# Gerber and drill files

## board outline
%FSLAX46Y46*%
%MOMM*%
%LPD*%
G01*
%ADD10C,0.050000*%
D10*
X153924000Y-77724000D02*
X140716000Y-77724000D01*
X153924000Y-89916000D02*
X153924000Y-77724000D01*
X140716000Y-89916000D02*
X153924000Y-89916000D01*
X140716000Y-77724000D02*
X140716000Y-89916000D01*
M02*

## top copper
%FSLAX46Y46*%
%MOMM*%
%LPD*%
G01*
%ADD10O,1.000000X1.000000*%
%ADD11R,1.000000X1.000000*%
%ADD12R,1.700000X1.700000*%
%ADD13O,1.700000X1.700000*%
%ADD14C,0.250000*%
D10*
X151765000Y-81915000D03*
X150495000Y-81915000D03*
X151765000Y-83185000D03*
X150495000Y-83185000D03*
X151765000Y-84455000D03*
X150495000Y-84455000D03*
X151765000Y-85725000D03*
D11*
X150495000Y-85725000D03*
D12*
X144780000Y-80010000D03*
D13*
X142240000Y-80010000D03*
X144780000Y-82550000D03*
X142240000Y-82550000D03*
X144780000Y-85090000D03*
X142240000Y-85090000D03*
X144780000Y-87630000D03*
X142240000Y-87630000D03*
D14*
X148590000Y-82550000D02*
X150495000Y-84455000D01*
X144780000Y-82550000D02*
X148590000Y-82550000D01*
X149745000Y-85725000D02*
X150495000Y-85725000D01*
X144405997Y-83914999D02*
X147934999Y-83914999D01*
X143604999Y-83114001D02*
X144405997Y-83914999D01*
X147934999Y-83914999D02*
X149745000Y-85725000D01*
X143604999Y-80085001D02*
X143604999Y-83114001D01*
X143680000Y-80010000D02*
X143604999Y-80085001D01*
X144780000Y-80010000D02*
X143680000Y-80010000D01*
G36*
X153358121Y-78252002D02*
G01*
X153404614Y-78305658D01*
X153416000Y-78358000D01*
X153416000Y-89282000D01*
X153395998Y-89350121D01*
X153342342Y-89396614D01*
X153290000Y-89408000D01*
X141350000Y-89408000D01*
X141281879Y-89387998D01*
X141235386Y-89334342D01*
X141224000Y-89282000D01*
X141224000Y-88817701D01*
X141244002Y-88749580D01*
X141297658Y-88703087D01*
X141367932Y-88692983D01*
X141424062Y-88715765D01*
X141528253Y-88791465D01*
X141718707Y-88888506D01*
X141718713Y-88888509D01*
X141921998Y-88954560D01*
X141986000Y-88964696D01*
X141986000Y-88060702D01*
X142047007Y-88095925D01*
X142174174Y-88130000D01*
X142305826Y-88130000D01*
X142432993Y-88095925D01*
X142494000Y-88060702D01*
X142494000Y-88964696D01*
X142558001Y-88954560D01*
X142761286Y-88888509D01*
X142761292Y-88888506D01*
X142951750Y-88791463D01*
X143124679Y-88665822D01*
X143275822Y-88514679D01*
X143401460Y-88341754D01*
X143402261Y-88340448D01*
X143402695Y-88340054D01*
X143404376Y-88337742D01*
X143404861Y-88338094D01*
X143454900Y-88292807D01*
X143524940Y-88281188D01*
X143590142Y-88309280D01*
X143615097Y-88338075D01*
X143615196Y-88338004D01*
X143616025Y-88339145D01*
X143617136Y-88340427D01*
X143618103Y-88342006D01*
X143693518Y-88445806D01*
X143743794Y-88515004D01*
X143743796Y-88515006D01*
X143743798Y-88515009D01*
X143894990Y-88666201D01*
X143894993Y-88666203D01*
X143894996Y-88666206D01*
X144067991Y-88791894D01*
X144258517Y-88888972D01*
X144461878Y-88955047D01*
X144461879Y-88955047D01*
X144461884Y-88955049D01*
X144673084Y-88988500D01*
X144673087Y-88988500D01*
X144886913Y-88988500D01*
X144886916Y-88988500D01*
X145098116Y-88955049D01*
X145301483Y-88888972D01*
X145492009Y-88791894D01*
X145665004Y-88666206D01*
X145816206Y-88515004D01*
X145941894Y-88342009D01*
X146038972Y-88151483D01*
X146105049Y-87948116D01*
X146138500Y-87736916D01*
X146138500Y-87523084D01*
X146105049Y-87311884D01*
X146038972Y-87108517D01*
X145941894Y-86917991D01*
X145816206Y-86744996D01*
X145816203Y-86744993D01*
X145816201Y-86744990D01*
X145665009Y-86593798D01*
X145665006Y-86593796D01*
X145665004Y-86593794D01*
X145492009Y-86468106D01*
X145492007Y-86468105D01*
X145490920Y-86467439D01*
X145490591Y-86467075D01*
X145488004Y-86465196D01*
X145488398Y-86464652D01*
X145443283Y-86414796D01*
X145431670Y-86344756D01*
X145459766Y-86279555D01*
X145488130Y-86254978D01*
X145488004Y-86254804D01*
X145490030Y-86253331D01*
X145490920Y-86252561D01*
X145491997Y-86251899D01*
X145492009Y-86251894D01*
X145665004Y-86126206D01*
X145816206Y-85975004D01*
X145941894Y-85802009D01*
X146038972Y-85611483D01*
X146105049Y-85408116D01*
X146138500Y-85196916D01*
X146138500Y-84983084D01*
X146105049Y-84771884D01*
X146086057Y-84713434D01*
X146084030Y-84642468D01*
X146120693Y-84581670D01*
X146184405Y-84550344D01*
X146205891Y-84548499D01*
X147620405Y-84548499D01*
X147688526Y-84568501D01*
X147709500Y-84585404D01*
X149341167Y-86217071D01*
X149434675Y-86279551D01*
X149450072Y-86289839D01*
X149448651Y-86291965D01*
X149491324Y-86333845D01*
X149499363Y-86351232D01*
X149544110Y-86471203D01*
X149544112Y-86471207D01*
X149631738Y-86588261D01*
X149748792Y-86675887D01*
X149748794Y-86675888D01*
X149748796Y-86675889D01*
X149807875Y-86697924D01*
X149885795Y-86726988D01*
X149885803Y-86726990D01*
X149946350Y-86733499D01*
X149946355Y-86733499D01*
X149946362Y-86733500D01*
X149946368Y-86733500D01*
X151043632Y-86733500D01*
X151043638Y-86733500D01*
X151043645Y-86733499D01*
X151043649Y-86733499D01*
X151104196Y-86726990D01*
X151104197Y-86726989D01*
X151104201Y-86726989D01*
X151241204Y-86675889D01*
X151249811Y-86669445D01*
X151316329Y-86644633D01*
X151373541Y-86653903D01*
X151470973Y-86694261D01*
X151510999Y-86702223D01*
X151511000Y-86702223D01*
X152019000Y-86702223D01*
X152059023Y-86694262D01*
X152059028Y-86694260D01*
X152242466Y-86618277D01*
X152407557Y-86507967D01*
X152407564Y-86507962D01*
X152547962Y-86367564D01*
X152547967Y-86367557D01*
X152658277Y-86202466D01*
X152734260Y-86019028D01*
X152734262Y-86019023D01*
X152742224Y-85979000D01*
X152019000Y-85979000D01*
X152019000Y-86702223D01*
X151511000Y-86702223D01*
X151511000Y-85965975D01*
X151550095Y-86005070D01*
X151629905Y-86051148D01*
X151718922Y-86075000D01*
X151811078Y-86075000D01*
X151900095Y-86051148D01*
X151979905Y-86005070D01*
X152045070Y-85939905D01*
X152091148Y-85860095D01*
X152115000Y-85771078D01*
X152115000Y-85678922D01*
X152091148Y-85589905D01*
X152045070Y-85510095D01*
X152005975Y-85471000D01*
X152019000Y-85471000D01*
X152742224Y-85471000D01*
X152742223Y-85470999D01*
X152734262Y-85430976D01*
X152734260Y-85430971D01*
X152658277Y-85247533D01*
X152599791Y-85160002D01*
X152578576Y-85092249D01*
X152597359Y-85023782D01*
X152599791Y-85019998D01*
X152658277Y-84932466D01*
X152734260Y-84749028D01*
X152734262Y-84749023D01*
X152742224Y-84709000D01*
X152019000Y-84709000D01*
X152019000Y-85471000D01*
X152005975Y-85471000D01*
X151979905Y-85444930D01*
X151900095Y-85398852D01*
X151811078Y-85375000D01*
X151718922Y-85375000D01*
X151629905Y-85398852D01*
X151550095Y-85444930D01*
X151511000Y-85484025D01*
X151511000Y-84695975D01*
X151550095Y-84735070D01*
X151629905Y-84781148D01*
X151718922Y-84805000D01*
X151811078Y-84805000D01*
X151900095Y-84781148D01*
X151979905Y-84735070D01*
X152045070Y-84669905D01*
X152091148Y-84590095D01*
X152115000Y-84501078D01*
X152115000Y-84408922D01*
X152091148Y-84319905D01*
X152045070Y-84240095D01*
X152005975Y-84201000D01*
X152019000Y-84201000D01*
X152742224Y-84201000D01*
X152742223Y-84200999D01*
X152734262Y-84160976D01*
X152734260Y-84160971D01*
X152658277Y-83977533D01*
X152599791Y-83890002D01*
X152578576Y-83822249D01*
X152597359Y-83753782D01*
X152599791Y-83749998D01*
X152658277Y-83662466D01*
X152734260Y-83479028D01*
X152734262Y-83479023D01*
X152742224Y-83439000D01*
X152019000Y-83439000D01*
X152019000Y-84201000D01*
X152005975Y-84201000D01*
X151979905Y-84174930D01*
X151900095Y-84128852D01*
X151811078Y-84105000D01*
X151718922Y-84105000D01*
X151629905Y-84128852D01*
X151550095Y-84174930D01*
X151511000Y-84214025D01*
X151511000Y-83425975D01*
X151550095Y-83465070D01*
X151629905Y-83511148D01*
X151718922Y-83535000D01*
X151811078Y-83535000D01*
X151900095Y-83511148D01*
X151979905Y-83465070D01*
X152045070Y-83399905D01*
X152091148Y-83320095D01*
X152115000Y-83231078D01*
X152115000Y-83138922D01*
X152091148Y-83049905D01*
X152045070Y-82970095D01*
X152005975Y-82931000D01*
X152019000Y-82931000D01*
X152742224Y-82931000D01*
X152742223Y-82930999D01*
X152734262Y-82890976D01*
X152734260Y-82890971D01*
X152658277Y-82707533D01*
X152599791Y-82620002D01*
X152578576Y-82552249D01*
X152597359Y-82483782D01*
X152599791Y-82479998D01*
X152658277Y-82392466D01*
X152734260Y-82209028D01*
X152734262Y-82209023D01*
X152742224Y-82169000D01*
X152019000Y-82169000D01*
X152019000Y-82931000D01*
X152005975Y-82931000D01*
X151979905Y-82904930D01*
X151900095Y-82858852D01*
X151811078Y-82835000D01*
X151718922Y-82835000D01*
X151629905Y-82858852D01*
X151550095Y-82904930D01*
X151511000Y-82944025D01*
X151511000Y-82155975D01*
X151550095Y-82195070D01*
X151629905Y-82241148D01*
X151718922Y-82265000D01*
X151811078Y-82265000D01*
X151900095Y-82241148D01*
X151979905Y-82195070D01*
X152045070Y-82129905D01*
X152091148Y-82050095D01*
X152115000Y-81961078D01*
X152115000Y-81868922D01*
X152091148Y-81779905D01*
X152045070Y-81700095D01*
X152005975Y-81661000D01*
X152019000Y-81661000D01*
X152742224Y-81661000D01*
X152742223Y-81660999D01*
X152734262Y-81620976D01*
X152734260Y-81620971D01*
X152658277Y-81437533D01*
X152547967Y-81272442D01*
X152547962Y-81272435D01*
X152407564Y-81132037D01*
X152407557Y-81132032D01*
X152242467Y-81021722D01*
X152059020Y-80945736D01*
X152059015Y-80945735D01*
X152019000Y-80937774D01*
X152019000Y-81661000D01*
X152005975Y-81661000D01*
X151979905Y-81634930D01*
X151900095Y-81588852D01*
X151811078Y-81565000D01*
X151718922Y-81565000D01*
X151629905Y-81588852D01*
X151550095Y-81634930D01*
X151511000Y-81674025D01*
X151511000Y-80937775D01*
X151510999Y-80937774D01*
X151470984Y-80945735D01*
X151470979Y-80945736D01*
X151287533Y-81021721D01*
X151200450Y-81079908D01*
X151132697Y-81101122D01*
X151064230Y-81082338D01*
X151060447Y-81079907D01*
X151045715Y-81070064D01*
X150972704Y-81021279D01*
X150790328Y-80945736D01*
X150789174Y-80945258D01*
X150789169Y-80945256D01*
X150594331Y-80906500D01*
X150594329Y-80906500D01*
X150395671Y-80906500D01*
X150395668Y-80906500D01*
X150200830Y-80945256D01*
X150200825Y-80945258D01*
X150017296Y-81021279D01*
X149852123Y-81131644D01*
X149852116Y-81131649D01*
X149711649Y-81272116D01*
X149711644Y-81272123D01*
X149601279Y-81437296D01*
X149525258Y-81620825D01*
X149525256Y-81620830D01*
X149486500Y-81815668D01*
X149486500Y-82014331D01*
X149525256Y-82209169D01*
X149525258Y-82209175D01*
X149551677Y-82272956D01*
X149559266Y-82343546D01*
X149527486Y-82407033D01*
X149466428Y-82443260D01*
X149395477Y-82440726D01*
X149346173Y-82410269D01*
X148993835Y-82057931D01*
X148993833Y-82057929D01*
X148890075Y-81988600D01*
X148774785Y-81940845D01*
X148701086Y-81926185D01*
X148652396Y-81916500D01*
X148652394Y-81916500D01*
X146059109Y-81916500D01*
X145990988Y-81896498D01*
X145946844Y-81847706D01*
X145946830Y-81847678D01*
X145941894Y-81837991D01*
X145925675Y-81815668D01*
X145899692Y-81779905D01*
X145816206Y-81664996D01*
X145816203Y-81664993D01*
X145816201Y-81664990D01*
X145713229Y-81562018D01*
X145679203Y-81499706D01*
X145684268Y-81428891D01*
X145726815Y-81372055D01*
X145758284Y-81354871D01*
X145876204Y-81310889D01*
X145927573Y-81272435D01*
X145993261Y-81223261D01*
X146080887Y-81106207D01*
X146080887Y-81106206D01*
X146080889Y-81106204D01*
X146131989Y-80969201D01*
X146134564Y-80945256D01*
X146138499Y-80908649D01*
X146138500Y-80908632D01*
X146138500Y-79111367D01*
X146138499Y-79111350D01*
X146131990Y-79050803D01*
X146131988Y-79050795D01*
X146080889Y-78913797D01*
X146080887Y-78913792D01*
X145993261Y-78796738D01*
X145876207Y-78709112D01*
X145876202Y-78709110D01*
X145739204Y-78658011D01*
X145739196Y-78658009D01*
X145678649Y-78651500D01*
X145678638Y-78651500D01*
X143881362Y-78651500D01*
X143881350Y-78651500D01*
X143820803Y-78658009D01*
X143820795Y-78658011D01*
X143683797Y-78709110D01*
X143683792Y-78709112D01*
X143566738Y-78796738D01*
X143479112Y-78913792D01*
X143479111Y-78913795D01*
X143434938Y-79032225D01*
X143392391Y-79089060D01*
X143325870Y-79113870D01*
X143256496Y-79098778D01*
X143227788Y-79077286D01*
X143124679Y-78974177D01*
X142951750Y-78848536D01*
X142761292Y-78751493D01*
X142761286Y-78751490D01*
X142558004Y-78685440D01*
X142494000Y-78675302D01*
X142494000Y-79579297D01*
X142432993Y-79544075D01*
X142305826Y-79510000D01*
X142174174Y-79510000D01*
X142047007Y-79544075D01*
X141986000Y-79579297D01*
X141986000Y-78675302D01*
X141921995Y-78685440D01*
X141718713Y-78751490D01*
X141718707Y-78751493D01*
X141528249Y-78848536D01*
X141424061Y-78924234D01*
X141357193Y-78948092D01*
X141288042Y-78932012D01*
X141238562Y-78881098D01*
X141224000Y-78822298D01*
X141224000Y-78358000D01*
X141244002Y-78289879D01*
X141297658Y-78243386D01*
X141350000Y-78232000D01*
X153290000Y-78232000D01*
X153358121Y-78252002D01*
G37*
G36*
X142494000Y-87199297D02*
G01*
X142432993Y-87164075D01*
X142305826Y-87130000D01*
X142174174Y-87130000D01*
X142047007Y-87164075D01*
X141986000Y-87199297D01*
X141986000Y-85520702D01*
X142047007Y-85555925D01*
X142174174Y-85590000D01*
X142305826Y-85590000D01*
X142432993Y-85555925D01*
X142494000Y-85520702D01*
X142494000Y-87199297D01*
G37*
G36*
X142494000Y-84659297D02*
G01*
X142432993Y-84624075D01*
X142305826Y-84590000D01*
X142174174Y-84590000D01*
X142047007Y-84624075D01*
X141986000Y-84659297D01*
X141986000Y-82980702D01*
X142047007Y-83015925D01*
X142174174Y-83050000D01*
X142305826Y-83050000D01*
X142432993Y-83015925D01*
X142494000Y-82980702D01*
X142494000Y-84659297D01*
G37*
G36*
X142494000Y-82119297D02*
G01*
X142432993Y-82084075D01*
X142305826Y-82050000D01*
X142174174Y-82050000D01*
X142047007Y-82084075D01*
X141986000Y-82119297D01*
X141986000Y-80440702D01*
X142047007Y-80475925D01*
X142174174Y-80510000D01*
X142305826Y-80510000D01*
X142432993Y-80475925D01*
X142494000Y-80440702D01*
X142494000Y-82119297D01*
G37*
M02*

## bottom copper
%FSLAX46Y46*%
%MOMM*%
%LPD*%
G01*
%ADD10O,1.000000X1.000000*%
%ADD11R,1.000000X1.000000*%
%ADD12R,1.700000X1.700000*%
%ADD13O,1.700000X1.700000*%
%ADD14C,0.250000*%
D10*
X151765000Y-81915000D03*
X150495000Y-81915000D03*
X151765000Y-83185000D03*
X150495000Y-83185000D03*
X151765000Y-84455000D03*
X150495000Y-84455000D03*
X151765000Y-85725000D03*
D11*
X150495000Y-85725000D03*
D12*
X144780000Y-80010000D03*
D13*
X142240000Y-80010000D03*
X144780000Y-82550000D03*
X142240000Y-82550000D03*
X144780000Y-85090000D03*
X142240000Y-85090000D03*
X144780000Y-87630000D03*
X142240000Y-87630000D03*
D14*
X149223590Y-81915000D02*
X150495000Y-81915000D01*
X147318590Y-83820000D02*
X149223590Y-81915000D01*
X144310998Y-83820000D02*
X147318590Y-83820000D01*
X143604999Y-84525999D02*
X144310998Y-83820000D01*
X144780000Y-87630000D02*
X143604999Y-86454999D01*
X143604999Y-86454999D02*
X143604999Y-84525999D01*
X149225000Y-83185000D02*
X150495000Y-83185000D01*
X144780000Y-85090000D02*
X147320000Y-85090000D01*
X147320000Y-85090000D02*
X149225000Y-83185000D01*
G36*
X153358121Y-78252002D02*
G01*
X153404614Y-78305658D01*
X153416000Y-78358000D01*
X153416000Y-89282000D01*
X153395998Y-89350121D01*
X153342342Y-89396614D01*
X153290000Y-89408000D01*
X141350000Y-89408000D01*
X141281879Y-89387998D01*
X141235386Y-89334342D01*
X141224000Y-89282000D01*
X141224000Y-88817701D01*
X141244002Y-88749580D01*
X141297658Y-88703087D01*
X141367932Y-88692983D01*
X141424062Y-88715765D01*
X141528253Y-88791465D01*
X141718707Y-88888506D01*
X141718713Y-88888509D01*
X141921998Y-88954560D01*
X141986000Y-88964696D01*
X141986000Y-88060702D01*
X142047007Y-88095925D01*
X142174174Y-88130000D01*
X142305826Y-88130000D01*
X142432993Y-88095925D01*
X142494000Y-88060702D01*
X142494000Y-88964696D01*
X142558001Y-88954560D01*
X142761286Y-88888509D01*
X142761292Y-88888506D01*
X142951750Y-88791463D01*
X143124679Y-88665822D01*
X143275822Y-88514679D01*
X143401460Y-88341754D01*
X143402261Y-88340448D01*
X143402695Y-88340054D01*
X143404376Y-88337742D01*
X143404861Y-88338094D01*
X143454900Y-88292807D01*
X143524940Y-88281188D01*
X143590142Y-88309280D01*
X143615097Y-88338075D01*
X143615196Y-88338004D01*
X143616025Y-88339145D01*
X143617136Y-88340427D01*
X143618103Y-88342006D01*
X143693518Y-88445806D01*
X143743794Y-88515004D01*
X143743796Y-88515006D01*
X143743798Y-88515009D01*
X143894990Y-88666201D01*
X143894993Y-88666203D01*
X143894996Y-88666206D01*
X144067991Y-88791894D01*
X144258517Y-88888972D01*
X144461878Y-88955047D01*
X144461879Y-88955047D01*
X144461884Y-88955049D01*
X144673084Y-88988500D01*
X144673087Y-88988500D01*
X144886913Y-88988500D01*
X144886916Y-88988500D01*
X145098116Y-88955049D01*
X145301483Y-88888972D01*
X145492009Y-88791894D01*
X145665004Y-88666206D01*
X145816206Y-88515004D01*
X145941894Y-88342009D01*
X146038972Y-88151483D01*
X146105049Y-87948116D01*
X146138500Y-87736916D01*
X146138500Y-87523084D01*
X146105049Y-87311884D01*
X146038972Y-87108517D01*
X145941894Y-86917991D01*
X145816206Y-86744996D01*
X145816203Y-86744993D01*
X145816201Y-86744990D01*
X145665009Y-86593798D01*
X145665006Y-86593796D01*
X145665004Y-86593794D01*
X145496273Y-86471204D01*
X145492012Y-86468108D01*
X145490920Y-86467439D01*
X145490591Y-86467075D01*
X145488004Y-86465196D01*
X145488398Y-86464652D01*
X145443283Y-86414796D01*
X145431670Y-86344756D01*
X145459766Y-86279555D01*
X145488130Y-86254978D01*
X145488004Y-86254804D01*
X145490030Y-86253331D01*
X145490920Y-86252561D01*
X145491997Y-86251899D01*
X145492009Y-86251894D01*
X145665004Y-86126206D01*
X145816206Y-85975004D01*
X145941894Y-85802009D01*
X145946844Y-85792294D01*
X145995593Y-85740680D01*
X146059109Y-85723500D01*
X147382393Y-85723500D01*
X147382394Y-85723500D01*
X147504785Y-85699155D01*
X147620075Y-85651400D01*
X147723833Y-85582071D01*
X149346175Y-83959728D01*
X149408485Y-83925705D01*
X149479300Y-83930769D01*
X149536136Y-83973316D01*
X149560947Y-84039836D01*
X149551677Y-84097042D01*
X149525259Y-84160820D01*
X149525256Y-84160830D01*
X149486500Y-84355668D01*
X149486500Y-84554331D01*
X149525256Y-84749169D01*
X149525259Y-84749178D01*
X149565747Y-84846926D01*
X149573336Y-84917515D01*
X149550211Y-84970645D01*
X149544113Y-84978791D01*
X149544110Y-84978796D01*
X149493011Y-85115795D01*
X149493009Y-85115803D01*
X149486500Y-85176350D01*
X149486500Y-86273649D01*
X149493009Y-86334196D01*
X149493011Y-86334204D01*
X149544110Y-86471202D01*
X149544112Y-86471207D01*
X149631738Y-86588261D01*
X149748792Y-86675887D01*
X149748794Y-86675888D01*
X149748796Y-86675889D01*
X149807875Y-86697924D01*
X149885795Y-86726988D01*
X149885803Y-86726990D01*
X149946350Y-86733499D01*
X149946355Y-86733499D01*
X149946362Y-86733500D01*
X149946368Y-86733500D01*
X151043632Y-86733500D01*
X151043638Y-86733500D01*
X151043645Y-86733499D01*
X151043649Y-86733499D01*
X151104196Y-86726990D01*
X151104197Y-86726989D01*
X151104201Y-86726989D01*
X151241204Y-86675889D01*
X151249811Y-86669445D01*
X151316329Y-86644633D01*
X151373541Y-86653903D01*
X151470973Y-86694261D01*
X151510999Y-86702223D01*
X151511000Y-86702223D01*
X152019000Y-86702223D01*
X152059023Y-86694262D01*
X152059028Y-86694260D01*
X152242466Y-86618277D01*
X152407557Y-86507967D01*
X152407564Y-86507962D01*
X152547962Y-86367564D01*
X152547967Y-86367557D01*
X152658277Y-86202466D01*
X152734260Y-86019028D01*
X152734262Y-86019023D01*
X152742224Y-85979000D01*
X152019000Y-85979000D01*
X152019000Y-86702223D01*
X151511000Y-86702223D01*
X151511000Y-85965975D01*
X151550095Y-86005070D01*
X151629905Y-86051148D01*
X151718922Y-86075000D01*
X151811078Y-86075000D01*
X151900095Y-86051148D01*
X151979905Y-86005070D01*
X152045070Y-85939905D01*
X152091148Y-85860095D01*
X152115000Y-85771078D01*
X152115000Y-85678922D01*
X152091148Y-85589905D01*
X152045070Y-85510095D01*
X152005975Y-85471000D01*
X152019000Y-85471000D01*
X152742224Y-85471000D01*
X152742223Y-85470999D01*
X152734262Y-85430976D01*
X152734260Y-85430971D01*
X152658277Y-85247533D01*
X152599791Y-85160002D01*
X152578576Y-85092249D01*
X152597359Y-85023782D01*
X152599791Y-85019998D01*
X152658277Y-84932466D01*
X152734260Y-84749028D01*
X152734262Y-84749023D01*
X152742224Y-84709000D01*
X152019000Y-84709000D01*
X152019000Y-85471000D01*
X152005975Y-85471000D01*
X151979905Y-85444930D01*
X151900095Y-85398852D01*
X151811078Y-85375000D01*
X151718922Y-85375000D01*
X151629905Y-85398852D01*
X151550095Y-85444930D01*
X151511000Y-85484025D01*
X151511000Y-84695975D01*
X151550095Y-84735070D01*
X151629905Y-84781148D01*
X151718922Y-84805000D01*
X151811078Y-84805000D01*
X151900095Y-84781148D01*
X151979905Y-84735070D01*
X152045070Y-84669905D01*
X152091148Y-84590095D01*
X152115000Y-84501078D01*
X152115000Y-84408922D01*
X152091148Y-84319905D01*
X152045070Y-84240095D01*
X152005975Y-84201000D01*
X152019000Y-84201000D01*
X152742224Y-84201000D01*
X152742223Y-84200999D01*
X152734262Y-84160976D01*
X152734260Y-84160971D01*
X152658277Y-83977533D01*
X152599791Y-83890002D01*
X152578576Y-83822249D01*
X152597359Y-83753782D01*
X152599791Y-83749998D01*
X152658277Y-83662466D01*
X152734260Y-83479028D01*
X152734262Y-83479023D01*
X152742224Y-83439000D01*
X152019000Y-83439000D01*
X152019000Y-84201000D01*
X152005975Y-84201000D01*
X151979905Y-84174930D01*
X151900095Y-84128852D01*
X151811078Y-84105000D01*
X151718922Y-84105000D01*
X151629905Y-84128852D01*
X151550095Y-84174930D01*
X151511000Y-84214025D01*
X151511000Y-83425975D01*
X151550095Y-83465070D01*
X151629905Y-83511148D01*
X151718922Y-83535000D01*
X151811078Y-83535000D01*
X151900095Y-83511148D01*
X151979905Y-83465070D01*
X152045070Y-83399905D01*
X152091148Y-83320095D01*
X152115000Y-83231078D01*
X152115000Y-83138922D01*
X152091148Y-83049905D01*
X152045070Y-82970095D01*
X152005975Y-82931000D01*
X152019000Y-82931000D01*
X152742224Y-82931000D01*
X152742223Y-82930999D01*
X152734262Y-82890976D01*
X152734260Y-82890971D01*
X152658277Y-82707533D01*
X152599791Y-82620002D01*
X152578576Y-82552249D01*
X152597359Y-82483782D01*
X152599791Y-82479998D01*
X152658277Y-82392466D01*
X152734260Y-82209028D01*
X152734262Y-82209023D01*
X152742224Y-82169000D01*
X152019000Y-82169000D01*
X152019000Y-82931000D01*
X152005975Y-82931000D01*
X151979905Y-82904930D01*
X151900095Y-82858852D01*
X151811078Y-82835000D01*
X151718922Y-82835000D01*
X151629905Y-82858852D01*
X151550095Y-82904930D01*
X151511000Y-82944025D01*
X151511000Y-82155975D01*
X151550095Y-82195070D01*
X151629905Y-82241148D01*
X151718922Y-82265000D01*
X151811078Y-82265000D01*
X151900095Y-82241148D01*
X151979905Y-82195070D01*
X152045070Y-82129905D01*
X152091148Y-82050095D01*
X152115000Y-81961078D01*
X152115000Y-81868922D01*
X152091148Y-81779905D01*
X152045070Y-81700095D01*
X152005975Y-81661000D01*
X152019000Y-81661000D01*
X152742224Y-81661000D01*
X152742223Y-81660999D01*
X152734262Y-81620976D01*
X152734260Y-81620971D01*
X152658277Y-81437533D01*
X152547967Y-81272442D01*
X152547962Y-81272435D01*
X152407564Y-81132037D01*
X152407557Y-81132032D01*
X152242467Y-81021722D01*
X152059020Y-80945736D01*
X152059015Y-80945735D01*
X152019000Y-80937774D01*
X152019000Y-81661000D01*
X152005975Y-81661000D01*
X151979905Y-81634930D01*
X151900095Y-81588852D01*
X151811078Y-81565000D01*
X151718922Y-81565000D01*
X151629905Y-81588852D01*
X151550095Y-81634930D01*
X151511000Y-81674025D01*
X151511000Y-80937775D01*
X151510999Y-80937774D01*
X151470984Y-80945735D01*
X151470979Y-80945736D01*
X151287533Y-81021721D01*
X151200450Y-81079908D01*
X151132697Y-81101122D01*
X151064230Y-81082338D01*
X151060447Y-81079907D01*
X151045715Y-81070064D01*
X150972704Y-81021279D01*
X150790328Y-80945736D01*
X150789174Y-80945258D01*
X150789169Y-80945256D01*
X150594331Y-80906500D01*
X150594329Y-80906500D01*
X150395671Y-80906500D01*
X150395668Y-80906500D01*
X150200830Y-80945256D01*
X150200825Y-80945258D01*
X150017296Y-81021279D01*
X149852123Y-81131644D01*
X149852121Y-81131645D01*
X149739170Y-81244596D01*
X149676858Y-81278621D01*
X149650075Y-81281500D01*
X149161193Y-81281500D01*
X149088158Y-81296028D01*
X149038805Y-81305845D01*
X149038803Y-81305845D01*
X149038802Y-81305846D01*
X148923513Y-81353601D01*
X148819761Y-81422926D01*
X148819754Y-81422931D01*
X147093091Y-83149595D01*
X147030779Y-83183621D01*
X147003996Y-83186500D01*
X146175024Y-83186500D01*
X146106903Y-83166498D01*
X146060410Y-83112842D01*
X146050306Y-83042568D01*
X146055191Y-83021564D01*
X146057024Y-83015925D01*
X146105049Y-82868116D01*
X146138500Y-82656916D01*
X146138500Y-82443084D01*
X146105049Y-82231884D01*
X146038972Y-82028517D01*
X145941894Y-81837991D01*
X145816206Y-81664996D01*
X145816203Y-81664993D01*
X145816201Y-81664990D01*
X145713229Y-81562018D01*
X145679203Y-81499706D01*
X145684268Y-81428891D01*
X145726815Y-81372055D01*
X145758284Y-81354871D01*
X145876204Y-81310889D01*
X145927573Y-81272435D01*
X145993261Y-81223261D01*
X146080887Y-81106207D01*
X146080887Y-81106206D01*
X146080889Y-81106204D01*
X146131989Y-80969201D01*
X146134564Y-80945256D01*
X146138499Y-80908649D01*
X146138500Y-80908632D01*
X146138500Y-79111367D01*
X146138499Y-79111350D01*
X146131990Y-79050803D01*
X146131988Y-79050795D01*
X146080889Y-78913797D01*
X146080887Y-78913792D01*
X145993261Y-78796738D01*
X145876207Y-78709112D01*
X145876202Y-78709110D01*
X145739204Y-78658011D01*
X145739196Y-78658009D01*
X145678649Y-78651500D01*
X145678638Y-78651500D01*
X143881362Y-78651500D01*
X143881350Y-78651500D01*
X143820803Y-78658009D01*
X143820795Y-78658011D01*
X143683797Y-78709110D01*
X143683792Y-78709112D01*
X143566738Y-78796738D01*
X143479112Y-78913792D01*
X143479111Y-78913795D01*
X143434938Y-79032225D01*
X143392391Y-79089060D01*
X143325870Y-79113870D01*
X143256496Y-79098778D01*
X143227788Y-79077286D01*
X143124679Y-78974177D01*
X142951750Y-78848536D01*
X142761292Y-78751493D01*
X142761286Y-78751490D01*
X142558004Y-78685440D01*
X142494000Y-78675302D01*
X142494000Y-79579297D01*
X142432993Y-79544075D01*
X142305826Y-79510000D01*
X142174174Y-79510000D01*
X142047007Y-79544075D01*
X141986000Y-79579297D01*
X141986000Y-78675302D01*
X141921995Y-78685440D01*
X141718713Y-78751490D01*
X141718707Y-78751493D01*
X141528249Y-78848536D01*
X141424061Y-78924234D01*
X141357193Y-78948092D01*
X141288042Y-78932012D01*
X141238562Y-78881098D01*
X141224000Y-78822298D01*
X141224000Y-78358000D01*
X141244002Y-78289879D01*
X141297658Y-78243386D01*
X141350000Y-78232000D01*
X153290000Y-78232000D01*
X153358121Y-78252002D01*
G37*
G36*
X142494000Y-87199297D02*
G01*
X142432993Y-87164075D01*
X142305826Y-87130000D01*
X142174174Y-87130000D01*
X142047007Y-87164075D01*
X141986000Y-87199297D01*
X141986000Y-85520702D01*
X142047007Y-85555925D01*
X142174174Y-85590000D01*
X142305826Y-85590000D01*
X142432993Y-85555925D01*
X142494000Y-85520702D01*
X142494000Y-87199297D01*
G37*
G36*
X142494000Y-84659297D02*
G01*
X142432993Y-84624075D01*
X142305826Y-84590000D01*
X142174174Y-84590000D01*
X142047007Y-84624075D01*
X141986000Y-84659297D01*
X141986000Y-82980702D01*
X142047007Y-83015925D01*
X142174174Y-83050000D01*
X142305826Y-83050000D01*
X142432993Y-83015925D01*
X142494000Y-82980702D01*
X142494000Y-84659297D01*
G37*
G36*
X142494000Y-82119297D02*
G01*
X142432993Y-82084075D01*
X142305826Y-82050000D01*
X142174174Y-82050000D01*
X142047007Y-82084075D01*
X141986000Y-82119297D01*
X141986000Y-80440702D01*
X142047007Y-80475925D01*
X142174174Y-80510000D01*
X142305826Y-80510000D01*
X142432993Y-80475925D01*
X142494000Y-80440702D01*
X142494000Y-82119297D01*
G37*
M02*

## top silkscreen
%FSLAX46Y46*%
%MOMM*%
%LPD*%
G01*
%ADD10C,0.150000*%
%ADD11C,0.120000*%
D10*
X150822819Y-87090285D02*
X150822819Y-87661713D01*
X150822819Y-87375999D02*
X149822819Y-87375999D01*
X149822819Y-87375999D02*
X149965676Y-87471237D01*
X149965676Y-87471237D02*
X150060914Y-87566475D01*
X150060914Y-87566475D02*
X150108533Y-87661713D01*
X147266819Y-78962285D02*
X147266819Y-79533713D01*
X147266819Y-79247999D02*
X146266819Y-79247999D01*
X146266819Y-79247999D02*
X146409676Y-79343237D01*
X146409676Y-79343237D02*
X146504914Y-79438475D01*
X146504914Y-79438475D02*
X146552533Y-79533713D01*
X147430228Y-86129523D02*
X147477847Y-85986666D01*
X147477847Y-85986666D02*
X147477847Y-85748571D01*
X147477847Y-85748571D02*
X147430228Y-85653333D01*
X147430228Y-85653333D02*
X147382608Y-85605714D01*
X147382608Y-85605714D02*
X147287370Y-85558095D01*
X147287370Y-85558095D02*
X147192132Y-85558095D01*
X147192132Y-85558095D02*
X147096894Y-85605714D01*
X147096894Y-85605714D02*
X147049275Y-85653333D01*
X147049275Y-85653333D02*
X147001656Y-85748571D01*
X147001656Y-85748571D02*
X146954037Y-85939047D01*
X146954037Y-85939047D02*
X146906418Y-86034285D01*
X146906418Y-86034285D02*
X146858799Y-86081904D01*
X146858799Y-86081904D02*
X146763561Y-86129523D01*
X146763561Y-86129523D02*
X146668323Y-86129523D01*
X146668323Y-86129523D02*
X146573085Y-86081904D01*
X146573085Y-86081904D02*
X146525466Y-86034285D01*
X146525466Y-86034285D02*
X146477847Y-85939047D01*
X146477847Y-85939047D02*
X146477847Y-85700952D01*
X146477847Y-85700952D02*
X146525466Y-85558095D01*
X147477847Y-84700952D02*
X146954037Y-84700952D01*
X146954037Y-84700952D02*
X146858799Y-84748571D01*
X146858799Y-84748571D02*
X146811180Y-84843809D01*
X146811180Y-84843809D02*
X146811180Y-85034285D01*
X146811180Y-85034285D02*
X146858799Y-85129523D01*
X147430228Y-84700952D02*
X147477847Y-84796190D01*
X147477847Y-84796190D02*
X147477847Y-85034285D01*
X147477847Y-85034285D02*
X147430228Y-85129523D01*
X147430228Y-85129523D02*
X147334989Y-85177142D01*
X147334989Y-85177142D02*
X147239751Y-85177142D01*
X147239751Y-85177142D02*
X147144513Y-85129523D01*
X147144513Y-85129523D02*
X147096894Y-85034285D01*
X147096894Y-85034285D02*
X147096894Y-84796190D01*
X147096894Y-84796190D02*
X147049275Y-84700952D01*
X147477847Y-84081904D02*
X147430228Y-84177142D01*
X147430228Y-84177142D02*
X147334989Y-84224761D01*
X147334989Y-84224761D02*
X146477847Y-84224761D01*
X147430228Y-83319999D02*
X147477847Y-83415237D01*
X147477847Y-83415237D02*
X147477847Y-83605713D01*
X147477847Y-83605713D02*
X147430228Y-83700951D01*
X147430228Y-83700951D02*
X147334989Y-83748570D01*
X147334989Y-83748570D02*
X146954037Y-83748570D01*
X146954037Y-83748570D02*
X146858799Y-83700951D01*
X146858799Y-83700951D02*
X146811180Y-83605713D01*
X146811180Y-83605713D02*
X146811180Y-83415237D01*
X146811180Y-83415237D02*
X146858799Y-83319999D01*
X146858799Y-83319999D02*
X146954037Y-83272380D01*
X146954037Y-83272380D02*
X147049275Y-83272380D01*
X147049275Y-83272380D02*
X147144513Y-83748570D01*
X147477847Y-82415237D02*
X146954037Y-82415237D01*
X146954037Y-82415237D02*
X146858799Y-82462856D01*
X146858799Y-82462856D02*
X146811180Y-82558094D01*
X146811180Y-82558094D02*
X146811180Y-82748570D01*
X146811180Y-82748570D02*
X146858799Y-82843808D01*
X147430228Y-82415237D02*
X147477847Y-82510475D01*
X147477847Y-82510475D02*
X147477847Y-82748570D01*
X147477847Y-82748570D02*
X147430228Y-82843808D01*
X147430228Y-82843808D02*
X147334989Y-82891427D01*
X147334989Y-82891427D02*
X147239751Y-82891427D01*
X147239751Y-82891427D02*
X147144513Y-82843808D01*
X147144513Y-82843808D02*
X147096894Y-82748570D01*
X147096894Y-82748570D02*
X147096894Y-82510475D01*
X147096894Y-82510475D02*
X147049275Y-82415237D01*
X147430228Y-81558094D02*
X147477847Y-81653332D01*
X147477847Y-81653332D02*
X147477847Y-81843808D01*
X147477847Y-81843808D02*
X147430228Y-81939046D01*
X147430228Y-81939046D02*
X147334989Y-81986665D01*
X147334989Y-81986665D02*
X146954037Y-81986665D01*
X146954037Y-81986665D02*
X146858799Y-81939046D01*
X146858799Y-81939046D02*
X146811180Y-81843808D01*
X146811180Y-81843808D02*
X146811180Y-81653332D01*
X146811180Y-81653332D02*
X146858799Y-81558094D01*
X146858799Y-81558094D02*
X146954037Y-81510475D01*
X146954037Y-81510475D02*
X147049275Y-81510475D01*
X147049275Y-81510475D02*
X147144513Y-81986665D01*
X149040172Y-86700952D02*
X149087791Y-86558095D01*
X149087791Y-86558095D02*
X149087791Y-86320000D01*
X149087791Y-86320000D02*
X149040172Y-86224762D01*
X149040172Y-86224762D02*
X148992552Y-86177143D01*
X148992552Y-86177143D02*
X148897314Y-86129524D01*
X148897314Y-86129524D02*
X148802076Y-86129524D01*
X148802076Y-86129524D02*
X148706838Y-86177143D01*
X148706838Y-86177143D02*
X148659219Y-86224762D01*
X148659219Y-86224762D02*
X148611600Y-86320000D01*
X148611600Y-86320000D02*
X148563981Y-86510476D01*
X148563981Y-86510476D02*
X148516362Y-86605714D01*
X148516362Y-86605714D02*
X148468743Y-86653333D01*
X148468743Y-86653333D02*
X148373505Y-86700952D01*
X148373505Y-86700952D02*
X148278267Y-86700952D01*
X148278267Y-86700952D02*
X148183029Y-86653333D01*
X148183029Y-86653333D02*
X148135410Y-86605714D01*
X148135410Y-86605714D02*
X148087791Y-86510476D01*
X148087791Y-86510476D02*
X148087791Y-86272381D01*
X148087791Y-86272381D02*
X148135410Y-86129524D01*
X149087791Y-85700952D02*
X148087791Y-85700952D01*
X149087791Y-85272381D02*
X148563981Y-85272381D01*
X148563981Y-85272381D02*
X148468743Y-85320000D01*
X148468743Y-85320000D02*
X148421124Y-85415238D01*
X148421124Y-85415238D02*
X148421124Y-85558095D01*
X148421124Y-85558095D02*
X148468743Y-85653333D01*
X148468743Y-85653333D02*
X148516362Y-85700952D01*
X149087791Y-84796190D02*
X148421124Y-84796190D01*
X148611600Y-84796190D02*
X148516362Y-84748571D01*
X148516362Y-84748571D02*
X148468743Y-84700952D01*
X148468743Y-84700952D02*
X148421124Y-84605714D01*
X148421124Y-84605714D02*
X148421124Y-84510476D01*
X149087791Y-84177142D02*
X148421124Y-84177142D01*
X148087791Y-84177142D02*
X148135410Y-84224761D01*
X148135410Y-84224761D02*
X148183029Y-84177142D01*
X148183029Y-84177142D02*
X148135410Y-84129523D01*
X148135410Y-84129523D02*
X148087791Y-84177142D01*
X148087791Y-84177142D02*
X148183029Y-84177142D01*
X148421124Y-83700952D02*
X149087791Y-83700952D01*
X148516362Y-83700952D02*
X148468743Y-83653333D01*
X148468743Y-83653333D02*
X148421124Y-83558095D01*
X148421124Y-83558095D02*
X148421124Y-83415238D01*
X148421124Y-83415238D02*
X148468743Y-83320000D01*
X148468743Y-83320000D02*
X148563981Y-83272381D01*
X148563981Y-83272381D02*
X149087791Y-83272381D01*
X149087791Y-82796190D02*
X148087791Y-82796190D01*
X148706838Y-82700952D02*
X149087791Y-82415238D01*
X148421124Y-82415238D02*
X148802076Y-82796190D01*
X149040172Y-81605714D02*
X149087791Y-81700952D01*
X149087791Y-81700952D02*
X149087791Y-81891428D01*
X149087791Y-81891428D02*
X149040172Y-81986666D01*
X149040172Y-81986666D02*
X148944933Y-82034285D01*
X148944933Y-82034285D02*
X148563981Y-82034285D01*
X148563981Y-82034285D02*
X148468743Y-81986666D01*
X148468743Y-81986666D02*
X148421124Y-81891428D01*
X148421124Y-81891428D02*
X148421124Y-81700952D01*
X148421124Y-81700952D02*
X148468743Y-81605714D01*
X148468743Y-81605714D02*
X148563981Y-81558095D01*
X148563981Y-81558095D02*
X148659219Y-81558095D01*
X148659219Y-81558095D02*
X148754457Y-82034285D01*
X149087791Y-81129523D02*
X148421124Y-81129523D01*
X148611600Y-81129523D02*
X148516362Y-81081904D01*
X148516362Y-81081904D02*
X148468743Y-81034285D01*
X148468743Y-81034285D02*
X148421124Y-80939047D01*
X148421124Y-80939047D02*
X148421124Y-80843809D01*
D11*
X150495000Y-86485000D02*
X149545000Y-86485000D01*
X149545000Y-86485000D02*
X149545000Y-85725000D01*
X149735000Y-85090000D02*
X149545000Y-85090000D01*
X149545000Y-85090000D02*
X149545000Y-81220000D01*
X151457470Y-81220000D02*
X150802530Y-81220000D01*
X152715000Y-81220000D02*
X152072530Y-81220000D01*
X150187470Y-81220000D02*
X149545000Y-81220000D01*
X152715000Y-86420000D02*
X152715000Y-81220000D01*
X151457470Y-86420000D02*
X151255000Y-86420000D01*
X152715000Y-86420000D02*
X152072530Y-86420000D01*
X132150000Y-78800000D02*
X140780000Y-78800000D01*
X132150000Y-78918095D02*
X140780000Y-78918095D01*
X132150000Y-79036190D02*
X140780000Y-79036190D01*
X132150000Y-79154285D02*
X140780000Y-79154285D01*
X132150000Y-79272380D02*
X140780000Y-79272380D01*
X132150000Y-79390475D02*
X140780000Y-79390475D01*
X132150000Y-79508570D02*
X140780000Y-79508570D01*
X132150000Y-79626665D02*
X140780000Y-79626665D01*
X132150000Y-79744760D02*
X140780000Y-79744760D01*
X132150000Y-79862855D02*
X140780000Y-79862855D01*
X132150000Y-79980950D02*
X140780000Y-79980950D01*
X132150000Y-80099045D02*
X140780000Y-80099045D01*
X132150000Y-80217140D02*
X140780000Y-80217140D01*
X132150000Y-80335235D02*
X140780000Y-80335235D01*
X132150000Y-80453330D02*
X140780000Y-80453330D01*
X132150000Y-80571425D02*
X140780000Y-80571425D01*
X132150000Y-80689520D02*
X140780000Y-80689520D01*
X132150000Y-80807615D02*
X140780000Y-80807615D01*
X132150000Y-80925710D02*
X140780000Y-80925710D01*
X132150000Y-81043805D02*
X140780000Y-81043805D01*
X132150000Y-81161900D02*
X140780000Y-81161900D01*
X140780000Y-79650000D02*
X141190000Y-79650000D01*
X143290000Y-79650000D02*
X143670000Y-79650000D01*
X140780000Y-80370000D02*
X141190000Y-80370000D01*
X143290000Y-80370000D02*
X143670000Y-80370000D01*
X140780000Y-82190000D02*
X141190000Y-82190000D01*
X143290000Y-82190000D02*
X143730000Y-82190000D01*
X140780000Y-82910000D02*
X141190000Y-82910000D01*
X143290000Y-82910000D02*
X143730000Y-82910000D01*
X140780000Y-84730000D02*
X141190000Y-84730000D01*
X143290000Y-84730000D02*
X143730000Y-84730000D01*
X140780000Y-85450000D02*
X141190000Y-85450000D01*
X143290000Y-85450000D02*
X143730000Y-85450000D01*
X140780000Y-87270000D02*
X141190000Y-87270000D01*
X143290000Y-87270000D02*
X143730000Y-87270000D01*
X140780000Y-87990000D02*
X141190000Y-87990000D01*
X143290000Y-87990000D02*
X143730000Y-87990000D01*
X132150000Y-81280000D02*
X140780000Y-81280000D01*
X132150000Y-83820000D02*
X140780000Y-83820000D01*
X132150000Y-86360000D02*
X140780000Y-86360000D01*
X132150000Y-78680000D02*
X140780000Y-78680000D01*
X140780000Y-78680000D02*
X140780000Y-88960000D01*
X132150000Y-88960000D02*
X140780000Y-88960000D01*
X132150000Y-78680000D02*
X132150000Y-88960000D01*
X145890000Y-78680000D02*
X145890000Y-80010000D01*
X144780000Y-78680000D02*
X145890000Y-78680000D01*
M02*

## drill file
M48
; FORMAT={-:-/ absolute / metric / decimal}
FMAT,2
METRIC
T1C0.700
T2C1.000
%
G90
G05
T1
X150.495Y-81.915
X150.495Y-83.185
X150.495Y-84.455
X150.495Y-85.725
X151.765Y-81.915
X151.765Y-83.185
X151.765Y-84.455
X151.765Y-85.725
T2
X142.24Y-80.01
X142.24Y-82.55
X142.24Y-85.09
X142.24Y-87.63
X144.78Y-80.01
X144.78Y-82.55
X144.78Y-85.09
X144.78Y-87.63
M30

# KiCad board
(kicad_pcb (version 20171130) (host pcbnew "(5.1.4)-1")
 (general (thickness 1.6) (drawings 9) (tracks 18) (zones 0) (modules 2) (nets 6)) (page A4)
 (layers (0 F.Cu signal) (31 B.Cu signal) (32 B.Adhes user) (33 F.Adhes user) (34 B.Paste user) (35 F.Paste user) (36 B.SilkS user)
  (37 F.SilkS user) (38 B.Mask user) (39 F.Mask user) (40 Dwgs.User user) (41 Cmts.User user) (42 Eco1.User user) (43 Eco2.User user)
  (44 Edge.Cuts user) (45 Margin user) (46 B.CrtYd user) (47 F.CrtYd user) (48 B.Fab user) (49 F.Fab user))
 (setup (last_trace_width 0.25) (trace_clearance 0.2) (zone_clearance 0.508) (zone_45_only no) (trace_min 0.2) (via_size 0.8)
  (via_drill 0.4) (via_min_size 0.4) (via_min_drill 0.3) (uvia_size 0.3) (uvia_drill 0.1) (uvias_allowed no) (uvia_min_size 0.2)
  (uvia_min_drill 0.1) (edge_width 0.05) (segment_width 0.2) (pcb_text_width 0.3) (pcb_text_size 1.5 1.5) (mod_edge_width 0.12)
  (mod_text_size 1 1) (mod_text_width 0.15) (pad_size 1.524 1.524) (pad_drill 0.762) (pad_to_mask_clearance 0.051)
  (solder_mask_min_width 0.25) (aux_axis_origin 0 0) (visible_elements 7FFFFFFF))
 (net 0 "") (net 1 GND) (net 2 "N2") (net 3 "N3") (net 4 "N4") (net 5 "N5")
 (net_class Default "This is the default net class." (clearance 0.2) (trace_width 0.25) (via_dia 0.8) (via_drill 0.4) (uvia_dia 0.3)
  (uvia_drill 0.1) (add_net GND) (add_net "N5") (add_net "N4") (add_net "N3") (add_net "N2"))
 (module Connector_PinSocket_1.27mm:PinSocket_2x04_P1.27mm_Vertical (layer F.Cu) (at 150.495 85.725 180)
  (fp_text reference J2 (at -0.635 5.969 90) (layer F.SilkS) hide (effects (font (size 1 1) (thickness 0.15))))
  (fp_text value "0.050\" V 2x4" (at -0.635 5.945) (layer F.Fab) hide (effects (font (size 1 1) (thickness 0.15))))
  (fp_line (start 0 -0.76) (end 0.95 -0.76) (layer F.SilkS) (width 0.12))
  (fp_line (start 0.95 -0.76) (end 0.95 0) (layer F.SilkS) (width 0.12))
  (fp_line (start 0.76 0.635) (end 0.95 0.635) (layer F.SilkS) (width 0.12))
  (fp_line (start 0.95 0.635) (end 0.95 4.505) (layer F.SilkS) (width 0.12))
  (fp_line (start -0.96247 4.505) (end -0.30753 4.505) (layer F.SilkS) (width 0.12))
  (fp_line (start -2.22 4.505) (end -1.57753 4.505) (layer F.SilkS) (width 0.12))
  (fp_line (start 0.30753 4.505) (end 0.95 4.505) (layer F.SilkS) (width 0.12))
  (fp_line (start -2.22 -0.695) (end -2.22 4.505) (layer F.SilkS) (width 0.12))
  (fp_line (start -0.96247 -0.695) (end -0.76 -0.695) (layer F.SilkS) (width 0.12))
  (fp_line (start -2.22 -0.695) (end -1.57753 -0.695) (layer F.SilkS) (width 0.12))
  (pad 8 thru_hole oval (at -1.27 3.81 180) (size 1 1) (drill 0.7) (layers *.Cu *.Mask) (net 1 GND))
  (pad 7 thru_hole oval (at 0 3.81 180) (size 1 1) (drill 0.7) (layers *.Cu *.Mask) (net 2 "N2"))
  (pad 6 thru_hole oval (at -1.27 2.54 180) (size 1 1) (drill 0.7) (layers *.Cu *.Mask) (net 1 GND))
  (pad 5 thru_hole oval (at 0 2.54 180) (size 1 1) (drill 0.7) (layers *.Cu *.Mask) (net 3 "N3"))
  (pad 4 thru_hole oval (at -1.27 1.27 180) (size 1 1) (drill 0.7) (layers *.Cu *.Mask) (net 1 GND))
  (pad 3 thru_hole oval (at 0 1.27 180) (size 1 1) (drill 0.7) (layers *.Cu *.Mask) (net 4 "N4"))
  (pad 2 thru_hole oval (at -1.27 0 180) (size 1 1) (drill 0.7) (layers *.Cu *.Mask) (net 1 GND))
  (pad 1 thru_hole rect (at 0 0 180) (size 1 1) (drill 0.7) (layers *.Cu *.Mask) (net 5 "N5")))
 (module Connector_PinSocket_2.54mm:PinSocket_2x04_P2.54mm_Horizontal (layer F.Cu) (at 144.78 80.01)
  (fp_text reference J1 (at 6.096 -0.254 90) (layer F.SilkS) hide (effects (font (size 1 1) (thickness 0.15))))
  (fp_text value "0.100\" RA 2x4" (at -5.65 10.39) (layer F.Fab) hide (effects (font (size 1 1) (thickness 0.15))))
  (fp_line (start -12.63 -1.21) (end -4 -1.21) (layer F.SilkS) (width 0.12))
  (fp_line (start -12.63 -1.091905) (end -4 -1.091905) (layer F.SilkS) (width 0.12))
  (fp_line (start -12.63 -0.97381) (end -4 -0.97381) (layer F.SilkS) (width 0.12))
  (fp_line (start -12.63 -0.855715) (end -4 -0.855715) (layer F.SilkS) (width 0.12))
  (fp_line (start -12.63 -0.73762) (end -4 -0.73762) (layer F.SilkS) (width 0.12))
  (fp_line (start -12.63 -0.619525) (end -4 -0.619525) (layer F.SilkS) (width 0.12))
  (fp_line (start -12.63 -0.50143) (end -4 -0.50143) (layer F.SilkS) (width 0.12))
  (fp_line (start -12.63 -0.383335) (end -4 -0.383335) (layer F.SilkS) (width 0.12))
  (fp_line (start -12.63 -0.26524) (end -4 -0.26524) (layer F.SilkS) (width 0.12))
  (fp_line (start -12.63 -0.147145) (end -4 -0.147145) (layer F.SilkS) (width 0.12))
  (fp_line (start -12.63 -0.02905) (end -4 -0.02905) (layer F.SilkS) (width 0.12))
  (fp_line (start -12.63 0.089045) (end -4 0.089045) (layer F.SilkS) (width 0.12))
  (fp_line (start -12.63 0.20714) (end -4 0.20714) (layer F.SilkS) (width 0.12))
  (fp_line (start -12.63 0.325235) (end -4 0.325235) (layer F.SilkS) (width 0.12))
  (fp_line (start -12.63 0.44333) (end -4 0.44333) (layer F.SilkS) (width 0.12))
  (fp_line (start -12.63 0.561425) (end -4 0.561425) (layer F.SilkS) (width 0.12))
  (fp_line (start -12.63 0.67952) (end -4 0.67952) (layer F.SilkS) (width 0.12))
  (fp_line (start -12.63 0.797615) (end -4 0.797615) (layer F.SilkS) (width 0.12))
  (fp_line (start -12.63 0.91571) (end -4 0.91571) (layer F.SilkS) (width 0.12))
  (fp_line (start -12.63 1.033805) (end -4 1.033805) (layer F.SilkS) (width 0.12))
  (fp_line (start -12.63 1.1519) (end -4 1.1519) (layer F.SilkS) (width 0.12))
  (fp_line (start -4 -0.36) (end -3.59 -0.36) (layer F.SilkS) (width 0.12))
  (fp_line (start -1.49 -0.36) (end -1.11 -0.36) (layer F.SilkS) (width 0.12))
  (fp_line (start -4 0.36) (end -3.59 0.36) (layer F.SilkS) (width 0.12))
  (fp_line (start -1.49 0.36) (end -1.11 0.36) (layer F.SilkS) (width 0.12))
  (fp_line (start -4 2.18) (end -3.59 2.18) (layer F.SilkS) (width 0.12))
  (fp_line (start -1.49 2.18) (end -1.05 2.18) (layer F.SilkS) (width 0.12))
  (fp_line (start -4 2.9) (end -3.59 2.9) (layer F.SilkS) (width 0.12))
  (fp_line (start -1.49 2.9) (end -1.05 2.9) (layer F.SilkS) (width 0.12))
  (fp_line (start -4 4.72) (end -3.59 4.72) (layer F.SilkS) (width 0.12))
  (fp_line (start -1.49 4.72) (end -1.05 4.72) (layer F.SilkS) (width 0.12))
  (fp_line (start -4 5.44) (end -3.59 5.44) (layer F.SilkS) (width 0.12))
  (fp_line (start -1.49 5.44) (end -1.05 5.44) (layer F.SilkS) (width 0.12))
  (fp_line (start -4 7.26) (end -3.59 7.26) (layer F.SilkS) (width 0.12))
  (fp_line (start -1.49 7.26) (end -1.05 7.26) (layer F.SilkS) (width 0.12))
  (fp_line (start -4 7.98) (end -3.59 7.98) (layer F.SilkS) (width 0.12))
  (fp_line (start -1.49 7.98) (end -1.05 7.98) (layer F.SilkS) (width 0.12))
  (fp_line (start -12.63 1.27) (end -4 1.27) (layer F.SilkS) (width 0.12))
  (fp_line (start -12.63 3.81) (end -4 3.81) (layer F.SilkS) (width 0.12))
  (fp_line (start -12.63 6.35) (end -4 6.35) (layer F.SilkS) (width 0.12))
  (fp_line (start -12.63 -1.33) (end -4 -1.33) (layer F.SilkS) (width 0.12))
  (fp_line (start -4 -1.33) (end -4 8.95) (layer F.SilkS) (width 0.12))
  (fp_line (start -12.63 8.95) (end -4 8.95) (layer F.SilkS) (width 0.12))
  (fp_line (start -12.63 -1.33) (end -12.63 8.95) (layer F.SilkS) (width 0.12))
  (fp_line (start 1.11 -1.33) (end 1.11 0) (layer F.SilkS) (width 0.12))
  (fp_line (start 0 -1.33) (end 1.11 -1.33) (layer F.SilkS) (width 0.12))
  (pad 1 thru_hole rect (at 0 0) (size 1.7 1.7) (drill 1) (layers *.Cu *.Mask) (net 5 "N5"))
  (pad 2 thru_hole oval (at -2.54 0) (size 1.7 1.7) (drill 1) (layers *.Cu *.Mask) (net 1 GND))
  (pad 3 thru_hole oval (at 0 2.54) (size 1.7 1.7) (drill 1) (layers *.Cu *.Mask) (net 4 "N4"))
  (pad 4 thru_hole oval (at -2.54 2.54) (size 1.7 1.7) (drill 1) (layers *.Cu *.Mask) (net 1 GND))
  (pad 5 thru_hole oval (at 0 5.08) (size 1.7 1.7) (drill 1) (layers *.Cu *.Mask) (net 3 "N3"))
  (pad 6 thru_hole oval (at -2.54 5.08) (size 1.7 1.7) (drill 1) (layers *.Cu *.Mask) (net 1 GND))
  (pad 7 thru_hole oval (at 0 7.62) (size 1.7 1.7) (drill 1) (layers *.Cu *.Mask) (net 2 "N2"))
  (pad 8 thru_hole oval (at -2.54 7.62) (size 1.7 1.7) (drill 1) (layers *.Cu *.Mask) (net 1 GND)))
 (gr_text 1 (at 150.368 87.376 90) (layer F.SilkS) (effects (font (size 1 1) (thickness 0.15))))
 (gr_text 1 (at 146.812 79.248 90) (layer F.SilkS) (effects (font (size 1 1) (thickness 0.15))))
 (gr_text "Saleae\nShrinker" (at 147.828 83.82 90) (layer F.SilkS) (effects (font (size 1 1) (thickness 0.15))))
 (gr_line (start 153.924 77.724) (end 140.716 77.724) (layer Edge.Cuts) (width 0.05))
 (gr_line (start 153.924 89.916) (end 153.924 77.724) (layer Edge.Cuts) (width 0.05))
 (gr_line (start 140.716 89.916) (end 153.924 89.916) (layer Edge.Cuts) (width 0.05))
 (gr_line (start 140.716 77.724) (end 140.716 89.916) (layer Edge.Cuts) (width 0.05))
 (segment (start 149.22359 81.915) (end 150.495 81.915) (width 0.25) (layer B.Cu) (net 2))
 (segment (start 147.31859 83.82) (end 149.22359 81.915) (width 0.25) (layer B.Cu) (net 2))
 (segment (start 144.310998 83.82) (end 147.31859 83.82) (width 0.25) (layer B.Cu) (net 2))
 (segment (start 143.604999 84.525999) (end 144.310998 83.82) (width 0.25) (layer B.Cu) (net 2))
 (segment (start 144.78 87.63) (end 143.604999 86.454999) (width 0.25) (layer B.Cu) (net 2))
 (segment (start 143.604999 86.454999) (end 143.604999 84.525999) (width 0.25) (layer B.Cu) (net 2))
 (segment (start 149.225 83.185) (end 150.495 83.185) (width 0.25) (layer B.Cu) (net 3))
 (segment (start 144.78 85.09) (end 147.32 85.09) (width 0.25) (layer B.Cu) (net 3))
 (segment (start 147.32 85.09) (end 149.225 83.185) (width 0.25) (layer B.Cu) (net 3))
 (segment (start 148.59 82.55) (end 150.495 84.455) (width 0.25) (layer F.Cu) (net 4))
 (segment (start 144.78 82.55) (end 148.59 82.55) (width 0.25) (layer F.Cu) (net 4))
 (segment (start 149.745 85.725) (end 150.495 85.725) (width 0.25) (layer F.Cu) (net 5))
 (segment (start 144.405997 83.914999) (end 147.934999 83.914999) (width 0.25) (layer F.Cu) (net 5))
 (segment (start 143.604999 83.114001) (end 144.405997 83.914999) (width 0.25) (layer F.Cu) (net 5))
 (segment (start 147.934999 83.914999) (end 149.745 85.725) (width 0.25) (layer F.Cu) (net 5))
 (segment (start 143.604999 80.085001) (end 143.604999 83.114001) (width 0.25) (layer F.Cu) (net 5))
 (segment (start 143.68 80.01) (end 143.604999 80.085001) (width 0.25) (layer F.Cu) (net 5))
 (segment (start 144.78 80.01) (end 143.68 80.01) (width 0.25) (layer F.Cu) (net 5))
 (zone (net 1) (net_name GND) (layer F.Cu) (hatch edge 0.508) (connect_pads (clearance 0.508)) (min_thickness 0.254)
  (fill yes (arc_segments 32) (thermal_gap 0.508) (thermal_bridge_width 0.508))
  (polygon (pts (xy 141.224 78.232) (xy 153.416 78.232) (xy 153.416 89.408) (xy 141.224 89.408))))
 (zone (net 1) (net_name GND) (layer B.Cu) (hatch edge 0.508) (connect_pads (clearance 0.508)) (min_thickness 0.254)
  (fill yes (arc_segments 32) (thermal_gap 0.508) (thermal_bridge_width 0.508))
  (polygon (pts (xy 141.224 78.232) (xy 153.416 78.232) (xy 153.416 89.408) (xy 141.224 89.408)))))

